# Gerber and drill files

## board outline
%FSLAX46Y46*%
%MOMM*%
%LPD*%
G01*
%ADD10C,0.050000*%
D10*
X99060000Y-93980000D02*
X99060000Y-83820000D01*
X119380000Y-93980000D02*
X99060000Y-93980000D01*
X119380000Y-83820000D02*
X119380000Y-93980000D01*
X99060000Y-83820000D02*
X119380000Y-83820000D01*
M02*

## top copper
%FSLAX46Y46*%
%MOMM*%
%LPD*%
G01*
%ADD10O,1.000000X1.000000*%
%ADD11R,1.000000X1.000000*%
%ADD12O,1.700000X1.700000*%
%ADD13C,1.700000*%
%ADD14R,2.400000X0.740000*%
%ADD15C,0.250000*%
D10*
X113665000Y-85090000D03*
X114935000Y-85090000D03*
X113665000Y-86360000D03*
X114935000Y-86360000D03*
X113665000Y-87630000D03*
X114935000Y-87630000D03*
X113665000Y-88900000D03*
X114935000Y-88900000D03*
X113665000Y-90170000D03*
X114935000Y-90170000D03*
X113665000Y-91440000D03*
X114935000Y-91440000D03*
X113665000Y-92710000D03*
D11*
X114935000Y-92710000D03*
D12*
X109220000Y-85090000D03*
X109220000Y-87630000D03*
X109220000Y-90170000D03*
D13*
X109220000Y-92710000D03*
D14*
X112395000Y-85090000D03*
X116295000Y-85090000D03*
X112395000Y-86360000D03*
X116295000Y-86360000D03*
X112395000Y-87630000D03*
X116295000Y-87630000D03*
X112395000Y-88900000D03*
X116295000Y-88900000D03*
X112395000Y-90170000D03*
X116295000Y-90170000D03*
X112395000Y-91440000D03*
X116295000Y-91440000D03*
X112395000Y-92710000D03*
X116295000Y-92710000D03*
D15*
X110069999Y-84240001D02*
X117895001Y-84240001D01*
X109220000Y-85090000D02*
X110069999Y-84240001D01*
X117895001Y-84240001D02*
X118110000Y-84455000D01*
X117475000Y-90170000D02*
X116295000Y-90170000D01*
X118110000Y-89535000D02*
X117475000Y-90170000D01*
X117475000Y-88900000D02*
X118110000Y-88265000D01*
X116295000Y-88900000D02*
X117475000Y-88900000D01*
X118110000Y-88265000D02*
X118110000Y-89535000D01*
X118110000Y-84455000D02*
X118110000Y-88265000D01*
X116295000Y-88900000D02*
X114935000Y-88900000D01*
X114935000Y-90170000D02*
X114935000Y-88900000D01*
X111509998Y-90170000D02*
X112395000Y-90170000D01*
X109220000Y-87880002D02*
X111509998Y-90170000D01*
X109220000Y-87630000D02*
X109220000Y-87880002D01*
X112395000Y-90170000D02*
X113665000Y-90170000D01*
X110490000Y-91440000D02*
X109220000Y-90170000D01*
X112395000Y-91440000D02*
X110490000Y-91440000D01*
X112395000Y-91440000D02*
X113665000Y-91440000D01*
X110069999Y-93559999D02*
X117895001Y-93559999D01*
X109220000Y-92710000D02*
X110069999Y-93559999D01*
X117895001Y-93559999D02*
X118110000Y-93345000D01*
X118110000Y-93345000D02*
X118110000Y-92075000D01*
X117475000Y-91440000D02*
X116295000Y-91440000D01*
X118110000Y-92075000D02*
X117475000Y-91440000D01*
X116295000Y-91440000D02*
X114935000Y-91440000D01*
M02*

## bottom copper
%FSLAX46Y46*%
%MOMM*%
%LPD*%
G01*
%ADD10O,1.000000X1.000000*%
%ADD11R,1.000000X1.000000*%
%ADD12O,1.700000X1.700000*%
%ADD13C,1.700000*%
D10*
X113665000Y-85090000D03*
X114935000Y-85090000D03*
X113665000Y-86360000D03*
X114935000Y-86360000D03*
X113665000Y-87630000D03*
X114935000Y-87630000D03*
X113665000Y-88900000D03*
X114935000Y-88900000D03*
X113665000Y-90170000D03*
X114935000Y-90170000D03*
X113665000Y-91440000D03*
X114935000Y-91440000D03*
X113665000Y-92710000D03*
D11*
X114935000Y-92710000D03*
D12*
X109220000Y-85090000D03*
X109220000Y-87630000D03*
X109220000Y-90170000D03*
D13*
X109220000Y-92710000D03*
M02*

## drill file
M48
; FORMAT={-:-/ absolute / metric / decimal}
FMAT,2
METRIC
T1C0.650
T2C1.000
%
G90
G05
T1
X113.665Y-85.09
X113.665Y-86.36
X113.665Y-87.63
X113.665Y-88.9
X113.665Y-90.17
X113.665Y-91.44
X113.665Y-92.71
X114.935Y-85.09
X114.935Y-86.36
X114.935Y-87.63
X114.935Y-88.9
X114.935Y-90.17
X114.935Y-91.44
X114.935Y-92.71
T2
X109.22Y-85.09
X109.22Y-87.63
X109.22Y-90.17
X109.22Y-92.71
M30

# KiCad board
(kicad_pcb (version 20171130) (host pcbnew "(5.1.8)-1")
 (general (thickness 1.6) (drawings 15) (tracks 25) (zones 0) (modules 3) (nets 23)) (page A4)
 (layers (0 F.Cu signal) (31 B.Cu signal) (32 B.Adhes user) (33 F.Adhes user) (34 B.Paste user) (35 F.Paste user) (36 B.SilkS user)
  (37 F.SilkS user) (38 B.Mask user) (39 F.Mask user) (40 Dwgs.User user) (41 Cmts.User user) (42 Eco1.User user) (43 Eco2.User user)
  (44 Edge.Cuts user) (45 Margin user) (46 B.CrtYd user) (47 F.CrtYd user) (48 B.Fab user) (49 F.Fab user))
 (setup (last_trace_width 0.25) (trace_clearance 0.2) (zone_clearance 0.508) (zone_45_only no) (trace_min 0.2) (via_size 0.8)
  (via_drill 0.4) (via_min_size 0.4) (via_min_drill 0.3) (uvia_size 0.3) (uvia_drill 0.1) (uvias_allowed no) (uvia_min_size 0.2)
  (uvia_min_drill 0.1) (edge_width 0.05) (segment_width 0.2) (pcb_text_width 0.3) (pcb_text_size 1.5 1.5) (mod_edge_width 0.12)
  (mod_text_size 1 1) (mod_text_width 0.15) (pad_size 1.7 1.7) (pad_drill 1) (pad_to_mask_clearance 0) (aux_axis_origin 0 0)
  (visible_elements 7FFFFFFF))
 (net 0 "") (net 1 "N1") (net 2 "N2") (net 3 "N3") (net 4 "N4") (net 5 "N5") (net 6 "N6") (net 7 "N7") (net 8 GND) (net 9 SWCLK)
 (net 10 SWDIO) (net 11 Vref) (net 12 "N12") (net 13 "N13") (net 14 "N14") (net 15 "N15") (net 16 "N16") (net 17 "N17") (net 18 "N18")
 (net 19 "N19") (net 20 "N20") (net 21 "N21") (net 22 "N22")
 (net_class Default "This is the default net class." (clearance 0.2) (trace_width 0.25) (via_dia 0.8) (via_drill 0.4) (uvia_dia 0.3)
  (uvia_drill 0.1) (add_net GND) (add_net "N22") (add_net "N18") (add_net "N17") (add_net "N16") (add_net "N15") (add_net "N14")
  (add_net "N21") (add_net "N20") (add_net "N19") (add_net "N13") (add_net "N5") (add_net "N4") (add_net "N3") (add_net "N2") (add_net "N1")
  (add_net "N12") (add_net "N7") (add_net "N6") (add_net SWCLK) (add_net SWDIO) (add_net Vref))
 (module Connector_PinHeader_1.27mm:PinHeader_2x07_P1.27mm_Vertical (layer F.Cu) (at 114.935 92.71 180)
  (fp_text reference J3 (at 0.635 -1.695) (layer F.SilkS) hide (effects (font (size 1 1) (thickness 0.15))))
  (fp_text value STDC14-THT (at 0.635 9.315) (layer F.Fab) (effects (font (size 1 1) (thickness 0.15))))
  (pad 14 thru_hole oval (at 1.27 7.62 180) (size 1 1) (drill 0.65) (layers *.Cu *.Mask) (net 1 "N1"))
  (pad 13 thru_hole oval (at 0 7.62 180) (size 1 1) (drill 0.65) (layers *.Cu *.Mask) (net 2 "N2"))
  (pad 12 thru_hole oval (at 1.27 6.35 180) (size 1 1) (drill 0.65) (layers *.Cu *.Mask) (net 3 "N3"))
  (pad 11 thru_hole oval (at 0 6.35 180) (size 1 1) (drill 0.65) (layers *.Cu *.Mask) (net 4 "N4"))
  (pad 10 thru_hole oval (at 1.27 5.08 180) (size 1 1) (drill 0.65) (layers *.Cu *.Mask) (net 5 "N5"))
  (pad 9 thru_hole oval (at 0 5.08 180) (size 1 1) (drill 0.65) (layers *.Cu *.Mask) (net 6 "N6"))
  (pad 8 thru_hole oval (at 1.27 3.81 180) (size 1 1) (drill 0.65) (layers *.Cu *.Mask) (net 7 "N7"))
  (pad 7 thru_hole oval (at 0 3.81 180) (size 1 1) (drill 0.65) (layers *.Cu *.Mask) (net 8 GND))
  (pad 6 thru_hole oval (at 1.27 2.54 180) (size 1 1) (drill 0.65) (layers *.Cu *.Mask) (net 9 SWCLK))
  (pad 5 thru_hole oval (at 0 2.54 180) (size 1 1) (drill 0.65) (layers *.Cu *.Mask) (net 8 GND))
  (pad 4 thru_hole oval (at 1.27 1.27 180) (size 1 1) (drill 0.65) (layers *.Cu *.Mask) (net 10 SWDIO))
  (pad 3 thru_hole oval (at 0 1.27 180) (size 1 1) (drill 0.65) (layers *.Cu *.Mask) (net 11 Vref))
  (pad 2 thru_hole oval (at 1.27 0 180) (size 1 1) (drill 0.65) (layers *.Cu *.Mask) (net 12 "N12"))
  (pad 1 thru_hole rect (at 0 0 180) (size 1 1) (drill 0.65) (layers *.Cu *.Mask) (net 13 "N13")))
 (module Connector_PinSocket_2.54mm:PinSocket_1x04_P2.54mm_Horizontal (layer B.Cu) (at 109.22 92.71)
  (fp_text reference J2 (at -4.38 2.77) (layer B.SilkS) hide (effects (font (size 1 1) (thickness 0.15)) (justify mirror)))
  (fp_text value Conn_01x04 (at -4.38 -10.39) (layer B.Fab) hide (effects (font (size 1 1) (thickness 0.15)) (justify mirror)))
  (pad 4 thru_hole oval (at 0 -7.62) (size 1.7 1.7) (drill 1) (layers *.Cu *.Mask) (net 8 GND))
  (pad 3 thru_hole oval (at 0 -5.08) (size 1.7 1.7) (drill 1) (layers *.Cu *.Mask) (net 9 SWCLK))
  (pad 2 thru_hole oval (at 0 -2.54) (size 1.7 1.7) (drill 1) (layers *.Cu *.Mask) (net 10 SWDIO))
  (pad 1 thru_hole circle (at 0 0) (size 1.7 1.7) (drill 1) (layers *.Cu *.Mask) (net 11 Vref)))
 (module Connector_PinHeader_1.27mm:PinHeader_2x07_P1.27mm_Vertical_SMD (layer F.Cu) (at 114.345 88.9 180)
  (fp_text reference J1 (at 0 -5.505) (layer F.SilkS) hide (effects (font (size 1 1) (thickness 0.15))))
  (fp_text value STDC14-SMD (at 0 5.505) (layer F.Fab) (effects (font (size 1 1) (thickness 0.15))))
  (pad 14 smd rect (at 1.95 3.81 180) (size 2.4 0.74) (layers F.Cu F.Paste F.Mask) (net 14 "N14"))
  (pad 13 smd rect (at -1.95 3.81 180) (size 2.4 0.74) (layers F.Cu F.Paste F.Mask) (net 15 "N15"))
  (pad 12 smd rect (at 1.95 2.54 180) (size 2.4 0.74) (layers F.Cu F.Paste F.Mask) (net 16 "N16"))
  (pad 11 smd rect (at -1.95 2.54 180) (size 2.4 0.74) (layers F.Cu F.Paste F.Mask) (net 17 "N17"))
  (pad 10 smd rect (at 1.95 1.27 180) (size 2.4 0.74) (layers F.Cu F.Paste F.Mask) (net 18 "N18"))
  (pad 9 smd rect (at -1.95 1.27 180) (size 2.4 0.74) (layers F.Cu F.Paste F.Mask) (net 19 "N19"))
  (pad 8 smd rect (at 1.95 0 180) (size 2.4 0.74) (layers F.Cu F.Paste F.Mask) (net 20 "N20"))
  (pad 7 smd rect (at -1.95 0 180) (size 2.4 0.74) (layers F.Cu F.Paste F.Mask) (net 8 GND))
  (pad 6 smd rect (at 1.95 -1.27 180) (size 2.4 0.74) (layers F.Cu F.Paste F.Mask) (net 9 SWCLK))
  (pad 5 smd rect (at -1.95 -1.27 180) (size 2.4 0.74) (layers F.Cu F.Paste F.Mask) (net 8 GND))
  (pad 4 smd rect (at 1.95 -2.54 180) (size 2.4 0.74) (layers F.Cu F.Paste F.Mask) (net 10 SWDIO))
  (pad 3 smd rect (at -1.95 -2.54 180) (size 2.4 0.74) (layers F.Cu F.Paste F.Mask) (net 11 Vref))
  (pad 2 smd rect (at 1.95 -3.81 180) (size 2.4 0.74) (layers F.Cu F.Paste F.Mask) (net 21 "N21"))
  (pad 1 smd rect (at -1.95 -3.81 180) (size 2.4 0.74) (layers F.Cu F.Paste F.Mask) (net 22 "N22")))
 (gr_line (start 99.06 93.98) (end 99.06 83.82) (layer Edge.Cuts) (width 0.05))
 (gr_line (start 119.38 93.98) (end 99.06 93.98) (layer Edge.Cuts) (width 0.05))
 (gr_line (start 119.38 83.82) (end 119.38 93.98) (layer Edge.Cuts) (width 0.05))
 (gr_line (start 99.06 83.82) (end 119.38 83.82) (layer Edge.Cuts) (width 0.05))
 (segment (start 110.069999 84.240001) (end 117.895001 84.240001) (width 0.25) (layer F.Cu) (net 8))
 (segment (start 109.22 85.09) (end 110.069999 84.240001) (width 0.25) (layer F.Cu) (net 8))
 (segment (start 117.895001 84.240001) (end 118.11 84.455) (width 0.25) (layer F.Cu) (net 8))
 (segment (start 117.475 90.17) (end 116.295 90.17) (width 0.25) (layer F.Cu) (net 8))
 (segment (start 118.11 89.535) (end 117.475 90.17) (width 0.25) (layer F.Cu) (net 8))
 (segment (start 117.475 88.9) (end 118.11 88.265) (width 0.25) (layer F.Cu) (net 8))
 (segment (start 116.295 88.9) (end 117.475 88.9) (width 0.25) (layer F.Cu) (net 8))
 (segment (start 118.11 88.265) (end 118.11 89.535) (width 0.25) (layer F.Cu) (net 8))
 (segment (start 118.11 84.455) (end 118.11 88.265) (width 0.25) (layer F.Cu) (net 8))
 (segment (start 116.295 88.9) (end 114.935 88.9) (width 0.25) (layer F.Cu) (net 8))
 (segment (start 114.935 90.17) (end 114.935 88.9) (width 0.25) (layer F.Cu) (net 8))
 (segment (start 111.509998 90.17) (end 112.395 90.17) (width 0.25) (layer F.Cu) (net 9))
 (segment (start 109.22 87.880002) (end 111.509998 90.17) (width 0.25) (layer F.Cu) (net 9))
 (segment (start 109.22 87.63) (end 109.22 87.880002) (width 0.25) (layer F.Cu) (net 9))
 (segment (start 112.395 90.17) (end 113.665 90.17) (width 0.25) (layer F.Cu) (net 9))
 (segment (start 110.49 91.44) (end 109.22 90.17) (width 0.25) (layer F.Cu) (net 10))
 (segment (start 112.395 91.44) (end 110.49 91.44) (width 0.25) (layer F.Cu) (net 10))
 (segment (start 112.395 91.44) (end 113.665 91.44) (width 0.25) (layer F.Cu) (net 10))
 (segment (start 110.069999 93.559999) (end 117.895001 93.559999) (width 0.25) (layer F.Cu) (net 11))
 (segment (start 109.22 92.71) (end 110.069999 93.559999) (width 0.25) (layer F.Cu) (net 11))
 (segment (start 117.895001 93.559999) (end 118.11 93.345) (width 0.25) (layer F.Cu) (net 11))
 (segment (start 118.11 93.345) (end 118.11 92.075) (width 0.25) (layer F.Cu) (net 11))
 (segment (start 117.475 91.44) (end 116.295 91.44) (width 0.25) (layer F.Cu) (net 11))
 (segment (start 118.11 92.075) (end 117.475 91.44) (width 0.25) (layer F.Cu) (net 11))
 (segment (start 116.295 91.44) (end 114.935 91.44) (width 0.25) (layer F.Cu) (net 11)))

